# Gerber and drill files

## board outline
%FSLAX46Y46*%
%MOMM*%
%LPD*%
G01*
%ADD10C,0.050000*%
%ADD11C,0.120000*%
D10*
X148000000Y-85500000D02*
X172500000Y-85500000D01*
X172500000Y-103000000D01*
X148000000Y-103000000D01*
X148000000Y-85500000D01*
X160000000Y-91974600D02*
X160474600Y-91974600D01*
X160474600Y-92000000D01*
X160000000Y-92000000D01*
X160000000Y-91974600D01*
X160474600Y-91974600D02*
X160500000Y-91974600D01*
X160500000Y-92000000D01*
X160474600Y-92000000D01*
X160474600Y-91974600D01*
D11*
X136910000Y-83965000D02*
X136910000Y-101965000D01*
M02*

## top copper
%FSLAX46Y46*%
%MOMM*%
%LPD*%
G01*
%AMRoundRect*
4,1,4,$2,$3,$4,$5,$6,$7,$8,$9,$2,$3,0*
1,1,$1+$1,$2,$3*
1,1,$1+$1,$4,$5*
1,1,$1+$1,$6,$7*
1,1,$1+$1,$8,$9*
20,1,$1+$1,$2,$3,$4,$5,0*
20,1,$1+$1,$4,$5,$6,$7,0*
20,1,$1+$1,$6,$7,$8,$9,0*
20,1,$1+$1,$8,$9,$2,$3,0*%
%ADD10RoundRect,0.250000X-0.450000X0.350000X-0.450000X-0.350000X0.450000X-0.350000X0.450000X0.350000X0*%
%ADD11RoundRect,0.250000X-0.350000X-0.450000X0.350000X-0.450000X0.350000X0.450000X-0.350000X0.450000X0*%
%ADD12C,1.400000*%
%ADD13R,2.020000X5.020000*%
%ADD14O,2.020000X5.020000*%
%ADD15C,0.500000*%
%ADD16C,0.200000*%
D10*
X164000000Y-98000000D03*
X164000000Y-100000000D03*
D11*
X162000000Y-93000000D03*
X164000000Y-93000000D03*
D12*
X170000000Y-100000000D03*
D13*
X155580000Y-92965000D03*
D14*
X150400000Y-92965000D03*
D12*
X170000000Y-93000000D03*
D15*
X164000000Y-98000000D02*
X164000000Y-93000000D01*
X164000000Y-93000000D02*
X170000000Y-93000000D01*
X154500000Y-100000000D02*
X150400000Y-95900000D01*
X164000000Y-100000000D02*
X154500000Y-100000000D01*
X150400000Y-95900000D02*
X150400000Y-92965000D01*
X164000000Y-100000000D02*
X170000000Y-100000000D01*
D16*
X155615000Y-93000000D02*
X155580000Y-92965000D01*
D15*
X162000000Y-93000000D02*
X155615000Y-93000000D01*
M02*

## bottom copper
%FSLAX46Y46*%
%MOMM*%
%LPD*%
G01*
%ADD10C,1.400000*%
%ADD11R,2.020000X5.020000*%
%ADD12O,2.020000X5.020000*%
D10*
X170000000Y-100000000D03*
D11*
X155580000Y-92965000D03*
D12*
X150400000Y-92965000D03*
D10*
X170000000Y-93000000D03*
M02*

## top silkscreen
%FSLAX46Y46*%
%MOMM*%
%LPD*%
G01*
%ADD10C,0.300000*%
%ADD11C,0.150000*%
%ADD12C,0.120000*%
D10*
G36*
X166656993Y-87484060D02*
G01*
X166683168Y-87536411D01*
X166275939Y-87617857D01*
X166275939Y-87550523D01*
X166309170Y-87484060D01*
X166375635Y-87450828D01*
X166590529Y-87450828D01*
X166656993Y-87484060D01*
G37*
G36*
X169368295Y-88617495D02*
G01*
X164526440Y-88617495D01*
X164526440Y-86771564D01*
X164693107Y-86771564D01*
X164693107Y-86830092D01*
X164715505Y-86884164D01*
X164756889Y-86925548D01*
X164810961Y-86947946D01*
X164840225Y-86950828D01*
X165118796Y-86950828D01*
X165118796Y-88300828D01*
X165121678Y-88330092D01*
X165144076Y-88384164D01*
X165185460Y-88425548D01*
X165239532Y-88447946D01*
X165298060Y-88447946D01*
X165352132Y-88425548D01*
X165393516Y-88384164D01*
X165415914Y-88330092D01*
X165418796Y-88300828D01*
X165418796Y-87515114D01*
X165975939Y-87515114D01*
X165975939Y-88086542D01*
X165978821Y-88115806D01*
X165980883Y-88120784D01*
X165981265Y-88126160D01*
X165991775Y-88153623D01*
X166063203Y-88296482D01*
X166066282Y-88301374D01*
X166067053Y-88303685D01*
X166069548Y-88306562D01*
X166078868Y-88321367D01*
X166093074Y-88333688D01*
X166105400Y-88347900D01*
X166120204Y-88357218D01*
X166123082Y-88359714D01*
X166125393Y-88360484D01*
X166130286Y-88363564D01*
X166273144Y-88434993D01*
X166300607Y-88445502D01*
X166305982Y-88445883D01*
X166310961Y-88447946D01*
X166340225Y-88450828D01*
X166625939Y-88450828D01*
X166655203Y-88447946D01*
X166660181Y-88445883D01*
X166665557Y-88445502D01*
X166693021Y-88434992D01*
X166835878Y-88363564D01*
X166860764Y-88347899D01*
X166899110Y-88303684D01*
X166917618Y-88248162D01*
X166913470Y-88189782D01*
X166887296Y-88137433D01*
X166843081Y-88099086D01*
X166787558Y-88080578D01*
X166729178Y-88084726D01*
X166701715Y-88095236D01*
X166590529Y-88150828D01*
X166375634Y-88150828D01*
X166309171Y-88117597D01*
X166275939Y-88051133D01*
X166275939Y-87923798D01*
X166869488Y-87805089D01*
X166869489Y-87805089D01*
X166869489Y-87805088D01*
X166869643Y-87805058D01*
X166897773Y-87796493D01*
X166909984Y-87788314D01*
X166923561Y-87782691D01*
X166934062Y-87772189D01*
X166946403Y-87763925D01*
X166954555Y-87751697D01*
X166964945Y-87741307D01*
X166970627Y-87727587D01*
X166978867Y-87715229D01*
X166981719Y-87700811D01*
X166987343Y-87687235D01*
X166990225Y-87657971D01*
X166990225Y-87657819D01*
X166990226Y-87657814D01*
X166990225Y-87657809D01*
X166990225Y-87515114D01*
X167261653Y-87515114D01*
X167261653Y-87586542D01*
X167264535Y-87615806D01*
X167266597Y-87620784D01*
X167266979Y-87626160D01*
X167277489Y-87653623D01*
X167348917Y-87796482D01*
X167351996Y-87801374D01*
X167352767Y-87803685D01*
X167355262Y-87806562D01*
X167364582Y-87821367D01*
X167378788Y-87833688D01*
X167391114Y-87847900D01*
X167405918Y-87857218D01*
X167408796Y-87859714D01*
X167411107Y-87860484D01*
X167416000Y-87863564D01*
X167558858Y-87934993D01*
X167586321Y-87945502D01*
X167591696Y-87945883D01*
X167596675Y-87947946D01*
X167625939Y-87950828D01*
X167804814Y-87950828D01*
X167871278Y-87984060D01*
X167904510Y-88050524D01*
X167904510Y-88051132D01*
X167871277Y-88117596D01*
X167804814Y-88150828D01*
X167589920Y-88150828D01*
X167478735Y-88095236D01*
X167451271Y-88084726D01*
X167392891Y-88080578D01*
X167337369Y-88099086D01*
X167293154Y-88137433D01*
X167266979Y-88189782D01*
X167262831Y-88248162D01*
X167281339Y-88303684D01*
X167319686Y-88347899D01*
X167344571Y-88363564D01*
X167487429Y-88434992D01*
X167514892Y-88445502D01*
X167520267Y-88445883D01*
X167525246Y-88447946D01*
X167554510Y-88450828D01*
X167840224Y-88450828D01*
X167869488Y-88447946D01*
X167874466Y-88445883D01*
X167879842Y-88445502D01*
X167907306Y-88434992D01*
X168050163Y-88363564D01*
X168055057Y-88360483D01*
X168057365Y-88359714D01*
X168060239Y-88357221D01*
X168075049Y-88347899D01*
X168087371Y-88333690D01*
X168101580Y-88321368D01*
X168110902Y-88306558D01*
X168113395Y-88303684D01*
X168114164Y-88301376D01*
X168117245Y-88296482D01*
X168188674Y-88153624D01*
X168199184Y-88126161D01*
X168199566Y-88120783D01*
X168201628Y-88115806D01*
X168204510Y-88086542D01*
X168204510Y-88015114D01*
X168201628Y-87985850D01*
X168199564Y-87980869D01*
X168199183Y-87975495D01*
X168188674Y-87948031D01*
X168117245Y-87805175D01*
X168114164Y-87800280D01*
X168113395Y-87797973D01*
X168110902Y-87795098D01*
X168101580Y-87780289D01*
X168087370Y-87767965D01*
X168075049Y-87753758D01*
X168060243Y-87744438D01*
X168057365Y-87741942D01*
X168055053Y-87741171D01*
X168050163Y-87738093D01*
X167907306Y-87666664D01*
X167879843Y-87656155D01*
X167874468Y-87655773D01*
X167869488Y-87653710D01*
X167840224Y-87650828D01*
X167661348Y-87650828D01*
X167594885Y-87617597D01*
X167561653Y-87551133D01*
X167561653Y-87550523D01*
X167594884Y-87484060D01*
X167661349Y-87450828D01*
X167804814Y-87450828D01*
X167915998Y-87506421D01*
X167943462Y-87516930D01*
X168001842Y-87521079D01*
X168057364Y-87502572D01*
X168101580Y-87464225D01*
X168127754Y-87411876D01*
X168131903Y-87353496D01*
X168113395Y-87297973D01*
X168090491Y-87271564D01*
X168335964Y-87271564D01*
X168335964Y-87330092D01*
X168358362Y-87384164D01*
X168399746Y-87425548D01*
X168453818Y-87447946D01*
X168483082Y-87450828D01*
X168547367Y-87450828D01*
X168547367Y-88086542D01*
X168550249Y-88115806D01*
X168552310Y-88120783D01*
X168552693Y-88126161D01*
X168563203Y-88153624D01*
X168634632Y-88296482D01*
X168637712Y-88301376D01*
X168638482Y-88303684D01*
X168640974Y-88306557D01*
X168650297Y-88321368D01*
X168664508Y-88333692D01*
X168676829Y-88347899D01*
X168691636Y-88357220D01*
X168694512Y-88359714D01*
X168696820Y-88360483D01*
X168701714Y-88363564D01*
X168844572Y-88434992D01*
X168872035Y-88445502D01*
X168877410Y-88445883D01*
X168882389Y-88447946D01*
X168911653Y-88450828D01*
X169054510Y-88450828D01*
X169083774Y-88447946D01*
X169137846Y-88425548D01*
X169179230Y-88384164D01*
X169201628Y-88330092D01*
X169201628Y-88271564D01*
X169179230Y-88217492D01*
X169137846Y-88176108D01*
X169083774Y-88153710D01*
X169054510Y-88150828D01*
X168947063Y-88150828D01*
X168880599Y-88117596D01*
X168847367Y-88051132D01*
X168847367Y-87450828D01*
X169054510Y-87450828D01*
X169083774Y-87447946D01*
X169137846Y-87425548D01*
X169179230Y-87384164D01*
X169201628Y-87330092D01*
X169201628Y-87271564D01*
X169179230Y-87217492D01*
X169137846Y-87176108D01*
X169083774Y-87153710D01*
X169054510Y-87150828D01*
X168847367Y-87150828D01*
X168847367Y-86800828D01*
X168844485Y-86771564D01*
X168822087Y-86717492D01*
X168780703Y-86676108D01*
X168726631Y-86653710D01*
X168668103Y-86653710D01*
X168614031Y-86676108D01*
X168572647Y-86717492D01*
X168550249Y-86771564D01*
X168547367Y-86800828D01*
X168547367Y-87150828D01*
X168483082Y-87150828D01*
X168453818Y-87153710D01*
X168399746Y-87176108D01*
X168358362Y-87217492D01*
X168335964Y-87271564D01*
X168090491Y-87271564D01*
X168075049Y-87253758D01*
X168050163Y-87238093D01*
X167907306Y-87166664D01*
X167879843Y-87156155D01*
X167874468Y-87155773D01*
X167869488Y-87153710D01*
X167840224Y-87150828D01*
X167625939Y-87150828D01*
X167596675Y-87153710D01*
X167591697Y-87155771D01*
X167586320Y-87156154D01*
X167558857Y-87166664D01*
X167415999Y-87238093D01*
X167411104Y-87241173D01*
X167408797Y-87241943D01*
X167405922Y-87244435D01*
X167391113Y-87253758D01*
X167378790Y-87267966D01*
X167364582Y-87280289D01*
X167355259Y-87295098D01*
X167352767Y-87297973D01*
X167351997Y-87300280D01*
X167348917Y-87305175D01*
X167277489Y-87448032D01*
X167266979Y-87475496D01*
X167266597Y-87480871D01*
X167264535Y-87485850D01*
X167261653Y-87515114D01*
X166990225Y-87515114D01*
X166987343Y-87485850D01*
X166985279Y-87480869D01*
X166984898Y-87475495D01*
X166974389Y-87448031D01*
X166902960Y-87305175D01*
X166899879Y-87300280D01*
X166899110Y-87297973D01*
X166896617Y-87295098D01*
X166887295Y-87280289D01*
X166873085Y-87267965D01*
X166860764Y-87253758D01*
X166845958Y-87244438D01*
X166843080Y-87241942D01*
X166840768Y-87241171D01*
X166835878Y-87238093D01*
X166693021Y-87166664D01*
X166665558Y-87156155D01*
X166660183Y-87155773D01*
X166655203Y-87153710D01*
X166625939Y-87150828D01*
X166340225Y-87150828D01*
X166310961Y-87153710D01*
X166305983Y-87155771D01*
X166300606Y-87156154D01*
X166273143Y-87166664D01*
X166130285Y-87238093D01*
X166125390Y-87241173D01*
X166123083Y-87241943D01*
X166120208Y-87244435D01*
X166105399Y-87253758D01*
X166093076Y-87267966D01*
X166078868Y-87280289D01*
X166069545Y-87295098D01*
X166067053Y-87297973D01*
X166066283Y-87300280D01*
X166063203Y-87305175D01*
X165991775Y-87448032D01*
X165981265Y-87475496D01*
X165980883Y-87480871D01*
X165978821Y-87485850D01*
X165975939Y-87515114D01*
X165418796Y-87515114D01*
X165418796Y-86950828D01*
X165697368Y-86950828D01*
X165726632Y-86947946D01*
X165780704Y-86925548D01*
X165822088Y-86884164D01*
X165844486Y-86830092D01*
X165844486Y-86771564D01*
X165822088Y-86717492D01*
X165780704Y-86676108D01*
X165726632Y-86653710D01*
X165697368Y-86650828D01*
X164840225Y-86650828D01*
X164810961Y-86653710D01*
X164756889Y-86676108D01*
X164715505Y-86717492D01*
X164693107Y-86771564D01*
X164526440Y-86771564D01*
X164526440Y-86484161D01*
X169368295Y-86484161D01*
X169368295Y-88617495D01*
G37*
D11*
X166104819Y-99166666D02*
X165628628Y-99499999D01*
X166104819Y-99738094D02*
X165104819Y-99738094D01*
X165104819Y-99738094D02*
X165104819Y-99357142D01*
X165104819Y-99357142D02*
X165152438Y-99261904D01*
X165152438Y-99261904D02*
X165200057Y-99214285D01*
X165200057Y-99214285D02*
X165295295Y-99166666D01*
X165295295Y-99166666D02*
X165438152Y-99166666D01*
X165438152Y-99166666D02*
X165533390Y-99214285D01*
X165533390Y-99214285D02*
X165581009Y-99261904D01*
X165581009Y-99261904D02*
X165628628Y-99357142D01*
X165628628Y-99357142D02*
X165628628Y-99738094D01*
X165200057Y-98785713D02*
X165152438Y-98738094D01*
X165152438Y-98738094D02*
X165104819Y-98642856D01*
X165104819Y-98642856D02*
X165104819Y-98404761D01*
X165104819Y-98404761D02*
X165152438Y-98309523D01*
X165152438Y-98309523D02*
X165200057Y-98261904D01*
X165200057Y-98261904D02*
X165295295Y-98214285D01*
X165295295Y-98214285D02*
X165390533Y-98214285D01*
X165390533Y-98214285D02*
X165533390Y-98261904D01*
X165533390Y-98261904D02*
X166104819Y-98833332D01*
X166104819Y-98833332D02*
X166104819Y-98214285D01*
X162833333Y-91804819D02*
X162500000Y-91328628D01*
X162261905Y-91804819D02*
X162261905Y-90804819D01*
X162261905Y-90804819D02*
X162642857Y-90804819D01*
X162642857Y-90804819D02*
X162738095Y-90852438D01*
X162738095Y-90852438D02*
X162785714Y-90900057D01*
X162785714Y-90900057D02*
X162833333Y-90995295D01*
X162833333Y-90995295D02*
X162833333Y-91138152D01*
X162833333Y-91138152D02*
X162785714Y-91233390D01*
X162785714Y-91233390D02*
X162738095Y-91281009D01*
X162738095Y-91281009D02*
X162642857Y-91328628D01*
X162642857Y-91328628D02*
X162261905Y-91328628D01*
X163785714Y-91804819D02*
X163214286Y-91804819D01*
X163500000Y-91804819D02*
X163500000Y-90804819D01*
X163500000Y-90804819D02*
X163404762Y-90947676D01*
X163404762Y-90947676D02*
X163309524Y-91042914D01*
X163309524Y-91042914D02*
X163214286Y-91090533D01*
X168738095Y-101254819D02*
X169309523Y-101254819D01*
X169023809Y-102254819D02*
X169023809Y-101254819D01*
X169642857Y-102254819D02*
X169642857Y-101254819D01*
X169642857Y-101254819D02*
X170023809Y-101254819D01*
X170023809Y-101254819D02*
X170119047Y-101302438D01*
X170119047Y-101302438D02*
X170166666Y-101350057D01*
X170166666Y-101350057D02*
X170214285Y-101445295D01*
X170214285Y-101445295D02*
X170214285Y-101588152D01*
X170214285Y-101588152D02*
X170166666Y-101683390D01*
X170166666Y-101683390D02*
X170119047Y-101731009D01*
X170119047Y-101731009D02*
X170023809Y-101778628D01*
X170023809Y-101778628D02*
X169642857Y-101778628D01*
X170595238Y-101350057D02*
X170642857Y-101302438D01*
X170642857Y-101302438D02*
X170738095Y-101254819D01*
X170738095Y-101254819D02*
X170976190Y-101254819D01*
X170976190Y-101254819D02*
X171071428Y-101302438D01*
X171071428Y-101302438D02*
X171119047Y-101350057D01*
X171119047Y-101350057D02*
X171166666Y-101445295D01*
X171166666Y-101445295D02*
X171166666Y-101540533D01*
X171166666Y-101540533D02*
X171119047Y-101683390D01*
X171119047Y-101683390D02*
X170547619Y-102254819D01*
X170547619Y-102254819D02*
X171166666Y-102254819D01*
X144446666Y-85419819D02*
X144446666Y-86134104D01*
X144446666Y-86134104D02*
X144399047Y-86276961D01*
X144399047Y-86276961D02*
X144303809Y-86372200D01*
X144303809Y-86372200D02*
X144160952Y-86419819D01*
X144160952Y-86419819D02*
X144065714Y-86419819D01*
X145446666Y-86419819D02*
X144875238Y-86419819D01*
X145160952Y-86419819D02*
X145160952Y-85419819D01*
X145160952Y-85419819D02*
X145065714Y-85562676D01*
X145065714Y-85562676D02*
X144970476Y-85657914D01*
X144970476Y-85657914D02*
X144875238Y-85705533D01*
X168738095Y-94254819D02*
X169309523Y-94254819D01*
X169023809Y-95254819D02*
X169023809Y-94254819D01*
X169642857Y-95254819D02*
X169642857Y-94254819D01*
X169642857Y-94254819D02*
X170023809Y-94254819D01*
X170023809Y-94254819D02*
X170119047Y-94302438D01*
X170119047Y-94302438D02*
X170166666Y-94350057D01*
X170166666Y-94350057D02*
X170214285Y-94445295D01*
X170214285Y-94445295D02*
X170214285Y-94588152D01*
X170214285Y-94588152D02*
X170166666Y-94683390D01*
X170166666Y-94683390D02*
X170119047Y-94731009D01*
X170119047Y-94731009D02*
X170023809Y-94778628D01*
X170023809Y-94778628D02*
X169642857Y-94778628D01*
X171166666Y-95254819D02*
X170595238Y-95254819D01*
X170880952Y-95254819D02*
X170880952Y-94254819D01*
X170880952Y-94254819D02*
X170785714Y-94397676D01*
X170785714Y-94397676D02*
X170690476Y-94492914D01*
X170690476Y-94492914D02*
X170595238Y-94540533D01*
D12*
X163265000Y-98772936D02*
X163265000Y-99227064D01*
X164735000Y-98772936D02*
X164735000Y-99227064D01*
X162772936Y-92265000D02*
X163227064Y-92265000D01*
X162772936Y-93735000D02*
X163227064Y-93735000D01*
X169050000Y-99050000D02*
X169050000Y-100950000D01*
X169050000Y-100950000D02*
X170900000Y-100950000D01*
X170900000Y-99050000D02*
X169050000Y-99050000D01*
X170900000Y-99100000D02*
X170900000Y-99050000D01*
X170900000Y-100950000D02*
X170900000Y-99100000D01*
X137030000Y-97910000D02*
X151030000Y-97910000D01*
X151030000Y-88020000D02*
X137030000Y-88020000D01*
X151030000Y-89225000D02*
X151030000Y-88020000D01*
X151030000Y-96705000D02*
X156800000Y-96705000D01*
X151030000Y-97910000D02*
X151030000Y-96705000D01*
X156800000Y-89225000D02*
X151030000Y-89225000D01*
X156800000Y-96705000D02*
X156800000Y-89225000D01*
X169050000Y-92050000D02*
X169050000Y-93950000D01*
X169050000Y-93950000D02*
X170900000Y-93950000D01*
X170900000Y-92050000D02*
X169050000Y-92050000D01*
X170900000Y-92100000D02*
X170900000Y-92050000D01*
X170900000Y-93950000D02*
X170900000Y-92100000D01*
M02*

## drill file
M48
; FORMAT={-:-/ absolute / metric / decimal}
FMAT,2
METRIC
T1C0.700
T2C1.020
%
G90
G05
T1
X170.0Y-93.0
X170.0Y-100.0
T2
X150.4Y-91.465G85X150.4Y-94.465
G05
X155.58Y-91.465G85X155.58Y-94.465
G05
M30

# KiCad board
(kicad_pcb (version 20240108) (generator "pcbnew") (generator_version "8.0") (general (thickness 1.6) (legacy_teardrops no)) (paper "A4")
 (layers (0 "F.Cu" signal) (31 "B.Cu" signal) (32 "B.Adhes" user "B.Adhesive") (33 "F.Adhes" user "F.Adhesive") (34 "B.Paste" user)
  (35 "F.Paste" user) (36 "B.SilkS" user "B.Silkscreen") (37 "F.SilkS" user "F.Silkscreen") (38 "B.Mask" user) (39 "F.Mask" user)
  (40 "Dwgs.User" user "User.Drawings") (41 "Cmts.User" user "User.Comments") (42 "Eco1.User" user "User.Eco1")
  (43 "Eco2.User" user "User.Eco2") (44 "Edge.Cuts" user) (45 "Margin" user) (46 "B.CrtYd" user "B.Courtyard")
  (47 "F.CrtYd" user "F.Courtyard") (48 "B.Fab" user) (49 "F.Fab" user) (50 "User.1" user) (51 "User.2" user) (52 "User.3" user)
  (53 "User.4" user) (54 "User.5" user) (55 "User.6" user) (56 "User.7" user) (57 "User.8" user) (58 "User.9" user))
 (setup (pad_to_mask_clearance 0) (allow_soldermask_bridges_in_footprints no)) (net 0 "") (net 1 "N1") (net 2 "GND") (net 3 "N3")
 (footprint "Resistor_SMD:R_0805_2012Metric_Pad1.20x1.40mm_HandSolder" (layer "F.Cu") (at 164 99 -90)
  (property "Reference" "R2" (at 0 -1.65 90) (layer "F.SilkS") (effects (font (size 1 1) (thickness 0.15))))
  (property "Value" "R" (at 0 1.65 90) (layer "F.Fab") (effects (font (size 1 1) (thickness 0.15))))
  (fp_line (start -0.227064 0.735) (end 0.227064 0.735) (stroke (width 0.12) (type solid)) (layer "F.SilkS"))
  (fp_line (start -0.227064 -0.735) (end 0.227064 -0.735) (stroke (width 0.12) (type solid)) (layer "F.SilkS"))
  (pad "1" smd roundrect (at -1 0 270) (size 1.2 1.4) (layers "F.Cu" "F.Paste" "F.Mask") (roundrect_rratio 0.208333) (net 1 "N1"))
  (pad "2" smd roundrect (at 1 0 270) (size 1.2 1.4) (layers "F.Cu" "F.Paste" "F.Mask") (roundrect_rratio 0.208333) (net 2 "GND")))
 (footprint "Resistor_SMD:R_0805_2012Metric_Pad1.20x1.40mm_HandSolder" (layer "F.Cu") (at 163 93)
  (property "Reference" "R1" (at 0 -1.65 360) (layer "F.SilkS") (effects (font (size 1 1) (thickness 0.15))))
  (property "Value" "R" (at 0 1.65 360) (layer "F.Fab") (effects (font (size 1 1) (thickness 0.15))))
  (fp_line (start -0.227064 -0.735) (end 0.227064 -0.735) (stroke (width 0.12) (type solid)) (layer "F.SilkS"))
  (fp_line (start -0.227064 0.735) (end 0.227064 0.735) (stroke (width 0.12) (type solid)) (layer "F.SilkS"))
  (pad "1" smd roundrect (at -1 0) (size 1.2 1.4) (layers "F.Cu" "F.Paste" "F.Mask") (roundrect_rratio 0.208333) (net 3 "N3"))
  (pad "2" smd roundrect (at 1 0) (size 1.2 1.4) (layers "F.Cu" "F.Paste" "F.Mask") (roundrect_rratio 0.208333) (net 1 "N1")))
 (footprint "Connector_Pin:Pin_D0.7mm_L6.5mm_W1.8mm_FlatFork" (layer "F.Cu") (at 170 100)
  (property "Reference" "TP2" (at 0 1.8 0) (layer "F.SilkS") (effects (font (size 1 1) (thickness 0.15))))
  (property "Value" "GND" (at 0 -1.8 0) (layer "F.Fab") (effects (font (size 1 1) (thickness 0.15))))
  (fp_line (start -0.95 -0.95) (end -0.95 0.95) (stroke (width 0.12) (type solid)) (layer "F.SilkS"))
  (fp_line (start -0.95 0.95) (end 0.9 0.95) (stroke (width 0.12) (type solid)) (layer "F.SilkS"))
  (fp_line (start 0.9 -0.95) (end -0.95 -0.95) (stroke (width 0.12) (type solid)) (layer "F.SilkS"))
  (fp_line (start 0.9 -0.9) (end 0.9 -0.95) (stroke (width 0.12) (type solid)) (layer "F.SilkS"))
  (fp_line (start 0.9 0.95) (end 0.9 -0.9) (stroke (width 0.12) (type solid)) (layer "F.SilkS"))
  (pad "1" thru_hole circle (at 0 0) (size 1.4 1.4) (drill 0.7) (layers "*.Cu" "*.Mask") (remove_unused_layers no) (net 2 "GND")))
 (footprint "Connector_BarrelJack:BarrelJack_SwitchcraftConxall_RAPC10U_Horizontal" (layer "F.Cu") (at 155.58 92.965)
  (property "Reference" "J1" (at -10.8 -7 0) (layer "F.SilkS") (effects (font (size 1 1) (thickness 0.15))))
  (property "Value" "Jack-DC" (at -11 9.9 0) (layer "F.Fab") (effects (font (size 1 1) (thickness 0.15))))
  (fp_line (start -18.55 4.945) (end -4.55 4.945) (stroke (width 0.12) (type solid)) (layer "F.SilkS"))
  (fp_line (start -4.55 -4.945) (end -18.55 -4.945) (stroke (width 0.12) (type solid)) (layer "F.SilkS"))
  (fp_line (start -4.55 -3.74) (end -4.55 -4.945) (stroke (width 0.12) (type solid)) (layer "F.SilkS"))
  (fp_line (start -4.55 3.74) (end 1.22 3.74) (stroke (width 0.12) (type solid)) (layer "F.SilkS"))
  (fp_line (start -4.55 4.945) (end -4.55 3.74) (stroke (width 0.12) (type solid)) (layer "F.SilkS"))
  (fp_line (start 1.22 -3.74) (end -4.55 -3.74) (stroke (width 0.12) (type solid)) (layer "F.SilkS"))
  (fp_line (start 1.22 3.74) (end 1.22 -3.74) (stroke (width 0.12) (type solid)) (layer "F.SilkS"))
  (fp_line (start -18.67 -9) (end -18.67 9) (stroke (width 0.12) (type solid)) (layer "Edge.Cuts"))
  (pad "1" thru_hole rect (at 0 0) (size 2.02 5.02) (drill oval 1.02 4.02) (layers "*.Cu" "*.Mask") (remove_unused_layers no) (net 3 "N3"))
  (pad "2" thru_hole oval (at -5.18 0) (size 2.02 5.02) (drill oval 1.02 4.02) (layers "*.Cu" "*.Mask") (remove_unused_layers no)
   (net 2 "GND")))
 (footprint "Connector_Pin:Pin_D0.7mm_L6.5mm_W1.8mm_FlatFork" (layer "F.Cu") (at 170 93)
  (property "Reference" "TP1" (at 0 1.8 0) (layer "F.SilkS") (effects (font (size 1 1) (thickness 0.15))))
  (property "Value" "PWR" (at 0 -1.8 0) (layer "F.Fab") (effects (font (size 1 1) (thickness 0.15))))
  (fp_line (start -0.95 -0.95) (end -0.95 0.95) (stroke (width 0.12) (type solid)) (layer "F.SilkS"))
  (fp_line (start -0.95 0.95) (end 0.9 0.95) (stroke (width 0.12) (type solid)) (layer "F.SilkS"))
  (fp_line (start 0.9 -0.95) (end -0.95 -0.95) (stroke (width 0.12) (type solid)) (layer "F.SilkS"))
  (fp_line (start 0.9 -0.9) (end 0.9 -0.95) (stroke (width 0.12) (type solid)) (layer "F.SilkS"))
  (fp_line (start 0.9 0.95) (end 0.9 -0.9) (stroke (width 0.12) (type solid)) (layer "F.SilkS"))
  (pad "1" thru_hole circle (at 0 0) (size 1.4 1.4) (drill 0.7) (layers "*.Cu" "*.Mask") (remove_unused_layers no) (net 1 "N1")))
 (gr_rect (start 148 85.5) (end 172.5 103) (stroke (width 0.05) (type default)) (fill none) (layer "Edge.Cuts"))
 (gr_rect (start 160 91.9746) (end 160.4746 92) (stroke (width 0.05) (type default)) (fill none) (layer "Edge.Cuts"))
 (gr_rect (start 160.4746 91.9746) (end 160.5 92) (stroke (width 0.05) (type default)) (fill none) (layer "Edge.Cuts"))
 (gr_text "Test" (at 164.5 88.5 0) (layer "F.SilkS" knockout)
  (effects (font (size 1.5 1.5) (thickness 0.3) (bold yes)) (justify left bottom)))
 (segment (start 164 98) (end 164 93) (width 0.5) (layer "F.Cu") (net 1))
 (segment (start 164 93) (end 170 93) (width 0.5) (layer "F.Cu") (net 1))
 (segment (start 154.5 100) (end 150.4 95.9) (width 0.5) (layer "F.Cu") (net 2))
 (segment (start 164 100) (end 154.5 100) (width 0.5) (layer "F.Cu") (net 2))
 (segment (start 150.4 95.9) (end 150.4 92.965) (width 0.5) (layer "F.Cu") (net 2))
 (segment (start 164 100) (end 170 100) (width 0.5) (layer "F.Cu") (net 2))
 (segment (start 155.615 93) (end 155.58 92.965) (width 0.2) (layer "F.Cu") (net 3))
 (segment (start 162 93) (end 155.615 93) (width 0.5) (layer "F.Cu") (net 3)))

